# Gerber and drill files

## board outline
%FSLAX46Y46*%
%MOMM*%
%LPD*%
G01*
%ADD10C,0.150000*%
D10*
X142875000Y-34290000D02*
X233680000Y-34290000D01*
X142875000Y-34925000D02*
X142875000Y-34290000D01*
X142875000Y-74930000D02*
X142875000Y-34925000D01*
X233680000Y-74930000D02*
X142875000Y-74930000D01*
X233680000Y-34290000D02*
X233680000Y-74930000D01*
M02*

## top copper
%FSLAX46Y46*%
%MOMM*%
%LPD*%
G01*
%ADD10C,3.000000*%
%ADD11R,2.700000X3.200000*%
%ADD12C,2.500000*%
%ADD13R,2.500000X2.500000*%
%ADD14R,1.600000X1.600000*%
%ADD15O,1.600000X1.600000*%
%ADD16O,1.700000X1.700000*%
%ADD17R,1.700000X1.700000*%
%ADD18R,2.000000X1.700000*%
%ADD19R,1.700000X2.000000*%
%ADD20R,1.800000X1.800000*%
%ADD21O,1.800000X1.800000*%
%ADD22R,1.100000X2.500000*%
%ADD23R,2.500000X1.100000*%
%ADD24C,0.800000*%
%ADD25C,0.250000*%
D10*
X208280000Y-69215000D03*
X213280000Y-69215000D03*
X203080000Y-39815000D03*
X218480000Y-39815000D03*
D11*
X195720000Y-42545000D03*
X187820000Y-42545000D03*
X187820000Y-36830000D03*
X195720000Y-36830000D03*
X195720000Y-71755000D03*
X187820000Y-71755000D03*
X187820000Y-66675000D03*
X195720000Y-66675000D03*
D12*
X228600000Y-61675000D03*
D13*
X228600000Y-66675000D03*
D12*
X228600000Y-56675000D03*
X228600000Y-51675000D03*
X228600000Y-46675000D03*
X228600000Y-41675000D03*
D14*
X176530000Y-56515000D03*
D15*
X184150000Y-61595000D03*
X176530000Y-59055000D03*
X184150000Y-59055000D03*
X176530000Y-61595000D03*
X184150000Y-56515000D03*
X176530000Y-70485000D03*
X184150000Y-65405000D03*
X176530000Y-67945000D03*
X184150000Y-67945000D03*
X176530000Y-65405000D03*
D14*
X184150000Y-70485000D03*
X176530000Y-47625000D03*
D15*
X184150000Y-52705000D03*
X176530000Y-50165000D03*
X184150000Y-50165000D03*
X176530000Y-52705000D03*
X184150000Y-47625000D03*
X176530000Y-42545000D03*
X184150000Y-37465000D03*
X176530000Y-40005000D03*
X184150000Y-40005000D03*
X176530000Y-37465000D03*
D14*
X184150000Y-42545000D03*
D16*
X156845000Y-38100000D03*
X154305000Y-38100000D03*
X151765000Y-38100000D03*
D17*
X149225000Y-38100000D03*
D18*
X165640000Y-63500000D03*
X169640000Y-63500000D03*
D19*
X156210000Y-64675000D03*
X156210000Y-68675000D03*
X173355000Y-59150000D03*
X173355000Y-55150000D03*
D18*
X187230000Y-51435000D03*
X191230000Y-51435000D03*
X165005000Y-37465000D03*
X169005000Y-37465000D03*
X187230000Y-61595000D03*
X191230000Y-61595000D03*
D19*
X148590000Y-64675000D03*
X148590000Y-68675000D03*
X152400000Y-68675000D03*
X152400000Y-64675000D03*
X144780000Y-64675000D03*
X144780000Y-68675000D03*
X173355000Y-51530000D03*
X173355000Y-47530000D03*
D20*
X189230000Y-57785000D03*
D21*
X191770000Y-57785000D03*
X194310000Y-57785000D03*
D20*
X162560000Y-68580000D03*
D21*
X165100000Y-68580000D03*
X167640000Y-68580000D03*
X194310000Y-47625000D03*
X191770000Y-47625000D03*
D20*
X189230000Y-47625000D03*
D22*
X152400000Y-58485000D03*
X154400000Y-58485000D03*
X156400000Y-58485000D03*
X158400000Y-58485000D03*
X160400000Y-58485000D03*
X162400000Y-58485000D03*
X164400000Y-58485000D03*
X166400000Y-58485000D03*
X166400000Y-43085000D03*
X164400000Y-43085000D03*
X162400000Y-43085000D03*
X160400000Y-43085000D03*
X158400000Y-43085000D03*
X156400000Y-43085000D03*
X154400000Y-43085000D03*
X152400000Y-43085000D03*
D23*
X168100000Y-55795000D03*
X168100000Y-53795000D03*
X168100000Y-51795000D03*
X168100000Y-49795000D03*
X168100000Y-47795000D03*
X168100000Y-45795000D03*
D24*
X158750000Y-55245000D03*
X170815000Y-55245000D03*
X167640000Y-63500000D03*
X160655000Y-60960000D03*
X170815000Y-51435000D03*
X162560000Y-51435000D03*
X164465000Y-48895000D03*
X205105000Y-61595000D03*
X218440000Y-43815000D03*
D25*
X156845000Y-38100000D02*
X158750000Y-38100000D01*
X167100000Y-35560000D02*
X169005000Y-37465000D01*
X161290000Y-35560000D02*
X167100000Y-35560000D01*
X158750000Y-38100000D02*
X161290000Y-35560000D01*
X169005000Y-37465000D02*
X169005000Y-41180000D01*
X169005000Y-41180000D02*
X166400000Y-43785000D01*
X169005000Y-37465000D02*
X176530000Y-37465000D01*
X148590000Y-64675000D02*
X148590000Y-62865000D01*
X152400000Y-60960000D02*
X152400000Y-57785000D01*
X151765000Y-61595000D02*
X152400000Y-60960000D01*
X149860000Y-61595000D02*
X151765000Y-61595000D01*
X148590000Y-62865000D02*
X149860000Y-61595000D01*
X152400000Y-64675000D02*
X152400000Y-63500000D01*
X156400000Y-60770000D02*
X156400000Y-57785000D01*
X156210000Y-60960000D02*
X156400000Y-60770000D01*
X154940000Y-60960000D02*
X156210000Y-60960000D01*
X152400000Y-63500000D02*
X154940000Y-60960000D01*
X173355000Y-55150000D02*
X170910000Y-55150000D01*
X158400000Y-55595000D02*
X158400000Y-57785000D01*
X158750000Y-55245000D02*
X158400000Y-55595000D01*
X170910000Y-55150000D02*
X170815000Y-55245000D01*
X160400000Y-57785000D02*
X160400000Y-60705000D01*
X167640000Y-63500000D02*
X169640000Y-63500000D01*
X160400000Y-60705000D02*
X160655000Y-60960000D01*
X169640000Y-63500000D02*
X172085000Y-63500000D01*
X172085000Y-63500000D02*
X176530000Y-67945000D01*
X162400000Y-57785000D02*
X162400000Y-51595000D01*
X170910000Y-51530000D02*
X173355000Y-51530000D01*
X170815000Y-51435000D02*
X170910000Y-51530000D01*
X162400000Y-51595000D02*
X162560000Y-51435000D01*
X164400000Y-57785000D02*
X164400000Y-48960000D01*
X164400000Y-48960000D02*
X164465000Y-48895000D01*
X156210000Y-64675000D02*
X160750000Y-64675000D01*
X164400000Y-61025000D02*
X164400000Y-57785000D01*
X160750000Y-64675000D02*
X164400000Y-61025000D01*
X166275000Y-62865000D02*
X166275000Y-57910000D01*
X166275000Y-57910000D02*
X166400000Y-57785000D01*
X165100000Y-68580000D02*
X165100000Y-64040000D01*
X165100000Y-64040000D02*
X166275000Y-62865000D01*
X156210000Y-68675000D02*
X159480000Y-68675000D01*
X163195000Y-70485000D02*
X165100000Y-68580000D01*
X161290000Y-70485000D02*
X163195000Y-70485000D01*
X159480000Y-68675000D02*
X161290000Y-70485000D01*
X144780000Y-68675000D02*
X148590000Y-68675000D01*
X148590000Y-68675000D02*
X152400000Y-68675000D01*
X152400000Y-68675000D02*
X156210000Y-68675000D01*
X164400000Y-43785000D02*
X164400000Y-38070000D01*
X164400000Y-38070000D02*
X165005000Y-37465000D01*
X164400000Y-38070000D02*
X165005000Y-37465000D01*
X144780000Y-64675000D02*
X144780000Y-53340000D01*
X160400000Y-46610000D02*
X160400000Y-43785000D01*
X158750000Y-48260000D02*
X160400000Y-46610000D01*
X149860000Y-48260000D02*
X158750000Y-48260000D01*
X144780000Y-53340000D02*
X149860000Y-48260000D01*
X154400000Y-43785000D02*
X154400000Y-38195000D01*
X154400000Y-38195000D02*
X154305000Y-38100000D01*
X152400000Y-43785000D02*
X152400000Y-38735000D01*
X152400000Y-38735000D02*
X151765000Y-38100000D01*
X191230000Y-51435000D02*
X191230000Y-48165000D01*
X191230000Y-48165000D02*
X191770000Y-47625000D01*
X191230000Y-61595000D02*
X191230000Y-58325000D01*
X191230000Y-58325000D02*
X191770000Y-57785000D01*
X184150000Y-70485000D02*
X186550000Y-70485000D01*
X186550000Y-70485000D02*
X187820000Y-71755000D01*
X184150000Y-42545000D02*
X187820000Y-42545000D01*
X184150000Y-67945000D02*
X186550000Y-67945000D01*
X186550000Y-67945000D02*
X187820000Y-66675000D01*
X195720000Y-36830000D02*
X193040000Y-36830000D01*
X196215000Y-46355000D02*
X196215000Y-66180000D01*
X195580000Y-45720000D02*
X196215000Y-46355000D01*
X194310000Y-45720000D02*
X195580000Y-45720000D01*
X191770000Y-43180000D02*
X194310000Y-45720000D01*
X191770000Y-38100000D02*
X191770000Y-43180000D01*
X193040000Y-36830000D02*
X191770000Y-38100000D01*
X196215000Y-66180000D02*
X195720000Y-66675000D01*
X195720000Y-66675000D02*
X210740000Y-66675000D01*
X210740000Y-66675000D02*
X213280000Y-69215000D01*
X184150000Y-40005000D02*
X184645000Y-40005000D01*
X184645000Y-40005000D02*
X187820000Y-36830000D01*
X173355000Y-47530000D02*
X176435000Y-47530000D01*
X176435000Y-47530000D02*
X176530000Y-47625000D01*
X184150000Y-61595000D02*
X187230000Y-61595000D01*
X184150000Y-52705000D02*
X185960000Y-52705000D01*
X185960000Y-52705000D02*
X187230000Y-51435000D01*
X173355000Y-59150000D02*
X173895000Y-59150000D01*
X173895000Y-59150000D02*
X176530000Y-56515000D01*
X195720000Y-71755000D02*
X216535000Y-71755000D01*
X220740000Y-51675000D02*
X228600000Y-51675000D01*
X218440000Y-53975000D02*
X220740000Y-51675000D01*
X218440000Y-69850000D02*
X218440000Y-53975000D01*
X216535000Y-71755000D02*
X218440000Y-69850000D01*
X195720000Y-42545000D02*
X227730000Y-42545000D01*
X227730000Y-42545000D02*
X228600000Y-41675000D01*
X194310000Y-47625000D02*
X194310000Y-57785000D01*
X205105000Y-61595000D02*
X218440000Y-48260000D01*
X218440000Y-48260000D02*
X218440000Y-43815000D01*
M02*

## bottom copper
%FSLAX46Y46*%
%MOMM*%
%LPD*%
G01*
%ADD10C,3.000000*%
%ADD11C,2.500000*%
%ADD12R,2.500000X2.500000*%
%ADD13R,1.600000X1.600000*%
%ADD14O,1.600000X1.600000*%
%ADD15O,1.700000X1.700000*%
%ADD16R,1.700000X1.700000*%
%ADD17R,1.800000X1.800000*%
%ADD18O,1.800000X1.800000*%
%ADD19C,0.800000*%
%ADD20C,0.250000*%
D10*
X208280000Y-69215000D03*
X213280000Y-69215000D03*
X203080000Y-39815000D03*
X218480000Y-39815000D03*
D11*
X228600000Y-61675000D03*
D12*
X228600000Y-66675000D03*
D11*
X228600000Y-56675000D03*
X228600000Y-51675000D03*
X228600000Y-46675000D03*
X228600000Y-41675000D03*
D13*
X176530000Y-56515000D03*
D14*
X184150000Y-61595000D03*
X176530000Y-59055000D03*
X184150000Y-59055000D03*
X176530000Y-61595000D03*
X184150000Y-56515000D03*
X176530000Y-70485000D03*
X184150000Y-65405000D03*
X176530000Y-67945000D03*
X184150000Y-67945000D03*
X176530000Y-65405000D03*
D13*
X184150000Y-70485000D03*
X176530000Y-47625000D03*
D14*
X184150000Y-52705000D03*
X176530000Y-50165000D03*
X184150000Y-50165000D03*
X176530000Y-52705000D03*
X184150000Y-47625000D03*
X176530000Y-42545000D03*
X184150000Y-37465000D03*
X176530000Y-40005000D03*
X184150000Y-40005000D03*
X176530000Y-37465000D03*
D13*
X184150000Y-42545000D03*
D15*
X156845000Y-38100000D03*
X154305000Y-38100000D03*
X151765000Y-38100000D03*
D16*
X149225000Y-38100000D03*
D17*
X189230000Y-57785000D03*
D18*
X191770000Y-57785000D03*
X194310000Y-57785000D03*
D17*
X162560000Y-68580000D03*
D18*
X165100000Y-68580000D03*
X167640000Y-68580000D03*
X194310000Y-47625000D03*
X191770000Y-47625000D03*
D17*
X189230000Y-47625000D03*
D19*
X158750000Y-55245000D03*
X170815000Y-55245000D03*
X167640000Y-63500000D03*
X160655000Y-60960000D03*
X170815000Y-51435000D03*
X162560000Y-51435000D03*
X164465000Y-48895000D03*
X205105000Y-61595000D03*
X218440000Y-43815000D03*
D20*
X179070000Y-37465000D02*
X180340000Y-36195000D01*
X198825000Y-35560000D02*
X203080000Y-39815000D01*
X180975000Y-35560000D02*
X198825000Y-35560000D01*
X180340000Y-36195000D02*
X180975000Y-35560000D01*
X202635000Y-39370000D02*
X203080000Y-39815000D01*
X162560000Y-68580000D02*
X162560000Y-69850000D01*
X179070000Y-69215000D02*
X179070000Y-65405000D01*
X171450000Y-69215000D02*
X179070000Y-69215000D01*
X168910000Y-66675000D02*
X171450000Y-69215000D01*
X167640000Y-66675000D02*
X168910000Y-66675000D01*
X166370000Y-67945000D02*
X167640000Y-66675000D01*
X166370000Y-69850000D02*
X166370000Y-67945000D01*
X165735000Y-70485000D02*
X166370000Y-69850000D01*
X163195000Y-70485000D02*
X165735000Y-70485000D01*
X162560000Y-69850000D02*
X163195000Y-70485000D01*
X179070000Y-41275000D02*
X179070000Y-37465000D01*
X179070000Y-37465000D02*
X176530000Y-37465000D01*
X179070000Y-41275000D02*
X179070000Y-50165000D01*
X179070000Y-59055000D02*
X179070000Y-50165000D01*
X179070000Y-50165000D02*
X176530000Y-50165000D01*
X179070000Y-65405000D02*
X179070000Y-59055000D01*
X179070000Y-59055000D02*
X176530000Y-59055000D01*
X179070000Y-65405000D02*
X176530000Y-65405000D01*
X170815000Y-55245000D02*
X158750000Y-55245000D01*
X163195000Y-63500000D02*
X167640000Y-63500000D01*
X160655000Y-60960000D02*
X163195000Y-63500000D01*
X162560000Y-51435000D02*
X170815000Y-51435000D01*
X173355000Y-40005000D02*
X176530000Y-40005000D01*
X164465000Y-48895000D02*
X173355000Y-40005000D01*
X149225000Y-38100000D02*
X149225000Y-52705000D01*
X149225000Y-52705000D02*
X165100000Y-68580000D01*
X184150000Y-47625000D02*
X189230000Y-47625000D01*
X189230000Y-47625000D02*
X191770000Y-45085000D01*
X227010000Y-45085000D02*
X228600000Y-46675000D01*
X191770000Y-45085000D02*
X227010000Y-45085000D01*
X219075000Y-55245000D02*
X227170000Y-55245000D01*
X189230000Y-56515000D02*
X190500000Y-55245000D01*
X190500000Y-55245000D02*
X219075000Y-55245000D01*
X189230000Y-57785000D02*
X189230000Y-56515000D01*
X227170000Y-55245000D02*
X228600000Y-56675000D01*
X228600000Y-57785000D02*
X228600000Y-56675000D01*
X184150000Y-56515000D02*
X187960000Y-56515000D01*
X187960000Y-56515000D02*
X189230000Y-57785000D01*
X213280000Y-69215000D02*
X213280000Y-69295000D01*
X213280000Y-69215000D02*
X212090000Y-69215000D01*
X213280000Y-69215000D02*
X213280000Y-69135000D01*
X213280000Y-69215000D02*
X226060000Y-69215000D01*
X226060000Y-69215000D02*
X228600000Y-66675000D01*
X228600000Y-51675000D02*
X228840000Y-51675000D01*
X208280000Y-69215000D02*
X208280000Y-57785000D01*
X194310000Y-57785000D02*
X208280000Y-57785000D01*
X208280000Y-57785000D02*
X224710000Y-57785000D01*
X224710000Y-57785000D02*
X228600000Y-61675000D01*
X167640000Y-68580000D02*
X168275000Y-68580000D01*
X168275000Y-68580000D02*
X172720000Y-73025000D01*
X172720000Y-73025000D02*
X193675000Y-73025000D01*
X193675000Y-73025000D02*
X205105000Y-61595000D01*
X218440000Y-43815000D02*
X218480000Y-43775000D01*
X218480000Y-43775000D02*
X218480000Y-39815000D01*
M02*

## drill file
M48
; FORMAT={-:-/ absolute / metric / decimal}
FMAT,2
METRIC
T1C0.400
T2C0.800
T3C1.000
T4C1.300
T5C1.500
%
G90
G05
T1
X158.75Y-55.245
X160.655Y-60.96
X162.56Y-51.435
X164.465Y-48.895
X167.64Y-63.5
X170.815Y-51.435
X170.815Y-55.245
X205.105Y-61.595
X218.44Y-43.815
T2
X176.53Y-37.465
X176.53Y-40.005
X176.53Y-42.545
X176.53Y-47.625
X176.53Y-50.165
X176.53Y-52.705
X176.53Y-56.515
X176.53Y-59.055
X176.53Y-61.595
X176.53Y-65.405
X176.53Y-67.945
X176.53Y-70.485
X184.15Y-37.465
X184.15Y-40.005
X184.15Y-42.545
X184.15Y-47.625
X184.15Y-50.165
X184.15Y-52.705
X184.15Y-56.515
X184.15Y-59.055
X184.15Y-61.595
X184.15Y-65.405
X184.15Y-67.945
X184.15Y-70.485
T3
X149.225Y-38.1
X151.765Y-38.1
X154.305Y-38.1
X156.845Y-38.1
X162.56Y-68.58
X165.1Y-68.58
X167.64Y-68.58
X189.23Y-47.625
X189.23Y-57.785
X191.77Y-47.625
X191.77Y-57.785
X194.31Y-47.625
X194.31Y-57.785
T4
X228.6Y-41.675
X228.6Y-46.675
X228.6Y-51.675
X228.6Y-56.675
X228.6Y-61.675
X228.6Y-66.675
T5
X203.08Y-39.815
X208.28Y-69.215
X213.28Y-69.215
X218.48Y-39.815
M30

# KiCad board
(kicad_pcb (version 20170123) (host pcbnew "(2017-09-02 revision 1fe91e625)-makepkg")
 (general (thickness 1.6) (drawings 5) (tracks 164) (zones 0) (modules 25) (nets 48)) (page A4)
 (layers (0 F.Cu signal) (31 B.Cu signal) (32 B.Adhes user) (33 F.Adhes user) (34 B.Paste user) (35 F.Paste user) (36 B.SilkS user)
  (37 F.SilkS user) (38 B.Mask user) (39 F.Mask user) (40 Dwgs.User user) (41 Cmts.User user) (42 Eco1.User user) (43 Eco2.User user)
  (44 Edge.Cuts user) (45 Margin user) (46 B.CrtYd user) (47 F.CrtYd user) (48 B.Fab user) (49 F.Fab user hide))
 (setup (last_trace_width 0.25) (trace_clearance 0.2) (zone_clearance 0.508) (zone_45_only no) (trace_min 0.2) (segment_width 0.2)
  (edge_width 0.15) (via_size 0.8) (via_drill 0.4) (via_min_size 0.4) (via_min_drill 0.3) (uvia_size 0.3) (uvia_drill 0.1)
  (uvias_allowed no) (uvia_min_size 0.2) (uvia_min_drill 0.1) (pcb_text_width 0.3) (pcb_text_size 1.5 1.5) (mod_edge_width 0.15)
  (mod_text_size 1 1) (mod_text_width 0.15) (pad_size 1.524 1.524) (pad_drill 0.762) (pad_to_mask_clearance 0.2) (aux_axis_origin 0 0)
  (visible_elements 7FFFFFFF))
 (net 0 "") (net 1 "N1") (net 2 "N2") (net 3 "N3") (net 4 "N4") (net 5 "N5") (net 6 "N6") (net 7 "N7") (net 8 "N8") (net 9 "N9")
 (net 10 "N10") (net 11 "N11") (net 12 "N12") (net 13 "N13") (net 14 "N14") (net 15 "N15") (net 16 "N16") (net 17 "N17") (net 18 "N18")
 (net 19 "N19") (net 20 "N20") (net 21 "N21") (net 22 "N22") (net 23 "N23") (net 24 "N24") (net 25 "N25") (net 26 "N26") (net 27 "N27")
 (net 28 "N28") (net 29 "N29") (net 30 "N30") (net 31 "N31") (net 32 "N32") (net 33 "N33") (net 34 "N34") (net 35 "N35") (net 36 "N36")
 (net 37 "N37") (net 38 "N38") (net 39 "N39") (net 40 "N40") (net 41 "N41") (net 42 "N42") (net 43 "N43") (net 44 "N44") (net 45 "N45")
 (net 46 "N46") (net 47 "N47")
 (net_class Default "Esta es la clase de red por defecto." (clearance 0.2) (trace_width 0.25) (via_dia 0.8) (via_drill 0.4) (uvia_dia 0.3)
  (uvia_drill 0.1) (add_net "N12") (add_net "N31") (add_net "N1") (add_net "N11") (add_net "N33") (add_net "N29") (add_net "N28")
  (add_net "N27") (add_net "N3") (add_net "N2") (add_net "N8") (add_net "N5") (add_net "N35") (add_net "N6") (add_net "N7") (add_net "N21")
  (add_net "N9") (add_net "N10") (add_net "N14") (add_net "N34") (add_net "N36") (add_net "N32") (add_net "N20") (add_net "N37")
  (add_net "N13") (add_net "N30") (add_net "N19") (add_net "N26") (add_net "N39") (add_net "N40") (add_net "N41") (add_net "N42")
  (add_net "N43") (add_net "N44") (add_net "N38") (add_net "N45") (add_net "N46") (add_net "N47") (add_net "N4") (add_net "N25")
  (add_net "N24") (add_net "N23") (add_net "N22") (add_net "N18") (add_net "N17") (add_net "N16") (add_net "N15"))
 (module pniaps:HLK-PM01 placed (layer F.Cu) (at 208.28 69.215 90)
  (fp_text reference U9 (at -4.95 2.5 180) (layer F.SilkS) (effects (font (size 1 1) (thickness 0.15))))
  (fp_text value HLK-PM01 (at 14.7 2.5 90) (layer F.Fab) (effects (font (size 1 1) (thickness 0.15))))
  (pad 1 thru_hole circle (at 0 0 90) (size 3 3) (drill 1.5) (layers *.Cu *.Mask F.SilkS) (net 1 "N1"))
  (pad 2 thru_hole circle (at 0 5 90) (size 3 3) (drill 1.5) (layers *.Cu *.Mask F.SilkS) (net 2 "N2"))
  (pad 4 thru_hole circle (at 29.4 -5.2 90) (size 3 3) (drill 1.5) (layers *.Cu *.Mask F.SilkS) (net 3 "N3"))
  (pad 3 thru_hole circle (at 29.4 10.2 90) (size 3 3) (drill 1.5) (layers *.Cu *.Mask F.SilkS) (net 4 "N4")))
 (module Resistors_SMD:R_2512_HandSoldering (layer F.Cu) (at 191.77 42.545 180)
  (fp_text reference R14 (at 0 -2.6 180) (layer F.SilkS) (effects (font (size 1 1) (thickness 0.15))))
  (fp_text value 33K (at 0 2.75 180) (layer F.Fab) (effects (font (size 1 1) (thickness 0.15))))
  (pad 1 smd rect (at -3.95 0 180) (size 2.7 3.2) (layers F.Cu F.Paste F.Mask) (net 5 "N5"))
  (pad 2 smd rect (at 3.95 0 180) (size 2.7 3.2) (layers F.Cu F.Paste F.Mask) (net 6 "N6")))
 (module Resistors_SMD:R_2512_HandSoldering (layer F.Cu) (at 191.77 36.83 180)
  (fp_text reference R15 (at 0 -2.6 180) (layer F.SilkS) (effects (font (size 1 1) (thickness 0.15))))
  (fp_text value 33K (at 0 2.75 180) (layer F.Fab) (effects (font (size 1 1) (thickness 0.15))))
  (pad 2 smd rect (at 3.95 0 180) (size 2.7 3.2) (layers F.Cu F.Paste F.Mask) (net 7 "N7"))
  (pad 1 smd rect (at -3.95 0 180) (size 2.7 3.2) (layers F.Cu F.Paste F.Mask) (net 2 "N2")))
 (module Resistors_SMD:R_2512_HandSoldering (layer F.Cu) (at 191.77 71.755 180)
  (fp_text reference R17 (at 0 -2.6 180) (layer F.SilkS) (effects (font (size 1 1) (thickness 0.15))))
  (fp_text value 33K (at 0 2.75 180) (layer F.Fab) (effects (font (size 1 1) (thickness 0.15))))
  (pad 1 smd rect (at -3.95 0 180) (size 2.7 3.2) (layers F.Cu F.Paste F.Mask) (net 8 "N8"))
  (pad 2 smd rect (at 3.95 0 180) (size 2.7 3.2) (layers F.Cu F.Paste F.Mask) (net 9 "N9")))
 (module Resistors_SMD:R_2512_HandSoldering (layer F.Cu) (at 191.77 66.675 180)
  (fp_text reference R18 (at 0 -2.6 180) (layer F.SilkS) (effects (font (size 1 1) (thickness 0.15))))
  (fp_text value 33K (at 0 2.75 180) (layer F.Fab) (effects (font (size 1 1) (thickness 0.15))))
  (pad 2 smd rect (at 3.95 0 180) (size 2.7 3.2) (layers F.Cu F.Paste F.Mask) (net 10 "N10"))
  (pad 1 smd rect (at -3.95 0 180) (size 2.7 3.2) (layers F.Cu F.Paste F.Mask) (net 2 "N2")))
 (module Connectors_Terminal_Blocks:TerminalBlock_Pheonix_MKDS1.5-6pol (layer F.Cu) (at 228.6 66.675 90)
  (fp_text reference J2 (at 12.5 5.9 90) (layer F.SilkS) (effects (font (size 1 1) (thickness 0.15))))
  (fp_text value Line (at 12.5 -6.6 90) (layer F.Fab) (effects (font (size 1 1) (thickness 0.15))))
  (pad 2 thru_hole circle (at 5 0 90) (size 2.5 2.5) (drill 1.3) (layers *.Cu *.Mask) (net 1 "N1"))
  (pad 1 thru_hole rect (at 0 0 90) (size 2.5 2.5) (drill 1.3) (layers *.Cu *.Mask) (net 2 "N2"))
  (pad 3 thru_hole circle (at 10 0 90) (size 2.5 2.5) (drill 1.3) (layers *.Cu *.Mask) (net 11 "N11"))
  (pad 4 thru_hole circle (at 15 0 90) (size 2.5 2.5) (drill 1.3) (layers *.Cu *.Mask) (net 8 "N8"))
  (pad 5 thru_hole circle (at 20 0 90) (size 2.5 2.5) (drill 1.3) (layers *.Cu *.Mask) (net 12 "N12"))
  (pad 6 thru_hole circle (at 25 0 90) (size 2.5 2.5) (drill 1.3) (layers *.Cu *.Mask) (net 5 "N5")))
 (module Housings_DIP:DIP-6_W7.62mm (layer F.Cu) (at 176.53 56.515)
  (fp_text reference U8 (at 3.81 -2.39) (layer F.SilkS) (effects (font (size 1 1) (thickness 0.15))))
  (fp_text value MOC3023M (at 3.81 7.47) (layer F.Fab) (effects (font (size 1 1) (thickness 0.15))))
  (pad 1 thru_hole rect (at 0 0) (size 1.6 1.6) (drill 0.8) (layers *.Cu *.Mask) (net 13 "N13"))
  (pad 4 thru_hole oval (at 7.62 5.08) (size 1.6 1.6) (drill 0.8) (layers *.Cu *.Mask) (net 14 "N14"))
  (pad 2 thru_hole oval (at 0 2.54) (size 1.6 1.6) (drill 0.8) (layers *.Cu *.Mask) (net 3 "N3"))
  (pad 5 thru_hole oval (at 7.62 2.54) (size 1.6 1.6) (drill 0.8) (layers *.Cu *.Mask) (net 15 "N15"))
  (pad 3 thru_hole oval (at 0 5.08) (size 1.6 1.6) (drill 0.8) (layers *.Cu *.Mask) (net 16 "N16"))
  (pad 6 thru_hole oval (at 7.62 0) (size 1.6 1.6) (drill 0.8) (layers *.Cu *.Mask) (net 11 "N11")))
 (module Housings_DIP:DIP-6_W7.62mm (layer F.Cu) (at 184.15 70.485 180)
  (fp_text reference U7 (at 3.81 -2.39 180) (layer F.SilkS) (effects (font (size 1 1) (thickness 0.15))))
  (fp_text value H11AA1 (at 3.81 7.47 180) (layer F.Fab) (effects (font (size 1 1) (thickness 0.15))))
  (pad 6 thru_hole oval (at 7.62 0 180) (size 1.6 1.6) (drill 0.8) (layers *.Cu *.Mask) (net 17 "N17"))
  (pad 3 thru_hole oval (at 0 5.08 180) (size 1.6 1.6) (drill 0.8) (layers *.Cu *.Mask) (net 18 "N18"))
  (pad 5 thru_hole oval (at 7.62 2.54 180) (size 1.6 1.6) (drill 0.8) (layers *.Cu *.Mask) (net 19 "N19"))
  (pad 2 thru_hole oval (at 0 2.54 180) (size 1.6 1.6) (drill 0.8) (layers *.Cu *.Mask) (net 10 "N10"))
  (pad 4 thru_hole oval (at 7.62 5.08 180) (size 1.6 1.6) (drill 0.8) (layers *.Cu *.Mask) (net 3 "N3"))
  (pad 1 thru_hole rect (at 0 0 180) (size 1.6 1.6) (drill 0.8) (layers *.Cu *.Mask) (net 9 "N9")))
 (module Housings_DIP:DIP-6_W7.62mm (layer F.Cu) (at 176.53 47.625)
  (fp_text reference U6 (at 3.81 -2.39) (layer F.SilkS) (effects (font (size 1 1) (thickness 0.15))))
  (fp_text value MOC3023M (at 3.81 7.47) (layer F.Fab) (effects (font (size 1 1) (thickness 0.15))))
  (pad 1 thru_hole rect (at 0 0) (size 1.6 1.6) (drill 0.8) (layers *.Cu *.Mask) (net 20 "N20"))
  (pad 4 thru_hole oval (at 7.62 5.08) (size 1.6 1.6) (drill 0.8) (layers *.Cu *.Mask) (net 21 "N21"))
  (pad 2 thru_hole oval (at 0 2.54) (size 1.6 1.6) (drill 0.8) (layers *.Cu *.Mask) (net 3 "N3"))
  (pad 5 thru_hole oval (at 7.62 2.54) (size 1.6 1.6) (drill 0.8) (layers *.Cu *.Mask) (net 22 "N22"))
  (pad 3 thru_hole oval (at 0 5.08) (size 1.6 1.6) (drill 0.8) (layers *.Cu *.Mask) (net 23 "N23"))
  (pad 6 thru_hole oval (at 7.62 0) (size 1.6 1.6) (drill 0.8) (layers *.Cu *.Mask) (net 12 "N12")))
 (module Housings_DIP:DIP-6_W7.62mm (layer F.Cu) (at 184.15 42.545 180)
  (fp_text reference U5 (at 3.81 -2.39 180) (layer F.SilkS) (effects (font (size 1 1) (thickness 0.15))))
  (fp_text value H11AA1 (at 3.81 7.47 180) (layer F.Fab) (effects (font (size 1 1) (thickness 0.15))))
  (pad 6 thru_hole oval (at 7.62 0 180) (size 1.6 1.6) (drill 0.8) (layers *.Cu *.Mask) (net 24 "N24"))
  (pad 3 thru_hole oval (at 0 5.08 180) (size 1.6 1.6) (drill 0.8) (layers *.Cu *.Mask) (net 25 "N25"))
  (pad 5 thru_hole oval (at 7.62 2.54 180) (size 1.6 1.6) (drill 0.8) (layers *.Cu *.Mask) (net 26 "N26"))
  (pad 2 thru_hole oval (at 0 2.54 180) (size 1.6 1.6) (drill 0.8) (layers *.Cu *.Mask) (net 7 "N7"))
  (pad 4 thru_hole oval (at 7.62 5.08 180) (size 1.6 1.6) (drill 0.8) (layers *.Cu *.Mask) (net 3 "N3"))
  (pad 1 thru_hole rect (at 0 0 180) (size 1.6 1.6) (drill 0.8) (layers *.Cu *.Mask) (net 6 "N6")))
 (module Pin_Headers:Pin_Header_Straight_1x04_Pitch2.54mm (layer F.Cu) (at 149.225 38.1 90)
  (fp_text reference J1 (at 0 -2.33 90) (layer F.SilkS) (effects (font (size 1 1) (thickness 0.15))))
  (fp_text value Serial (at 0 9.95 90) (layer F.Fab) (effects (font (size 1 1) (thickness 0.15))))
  (pad 4 thru_hole oval (at 0 7.62 90) (size 1.7 1.7) (drill 1) (layers *.Cu *.Mask) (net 3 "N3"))
  (pad 3 thru_hole oval (at 0 5.08 90) (size 1.7 1.7) (drill 1) (layers *.Cu *.Mask) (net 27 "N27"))
  (pad 2 thru_hole oval (at 0 2.54 90) (size 1.7 1.7) (drill 1) (layers *.Cu *.Mask) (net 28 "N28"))
  (pad 1 thru_hole rect (at 0 0 90) (size 1.7 1.7) (drill 1) (layers *.Cu *.Mask) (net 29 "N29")))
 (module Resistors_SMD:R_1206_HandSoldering (layer F.Cu) (at 167.64 63.5 180)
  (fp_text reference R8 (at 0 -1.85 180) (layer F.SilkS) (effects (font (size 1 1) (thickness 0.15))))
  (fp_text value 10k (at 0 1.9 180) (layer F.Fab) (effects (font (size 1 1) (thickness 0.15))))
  (pad 2 smd rect (at 2 0 180) (size 2 1.7) (layers F.Cu F.Paste F.Mask) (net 29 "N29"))
  (pad 1 smd rect (at -2 0 180) (size 2 1.7) (layers F.Cu F.Paste F.Mask) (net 19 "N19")))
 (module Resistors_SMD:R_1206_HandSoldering (layer F.Cu) (at 156.21 66.675 270)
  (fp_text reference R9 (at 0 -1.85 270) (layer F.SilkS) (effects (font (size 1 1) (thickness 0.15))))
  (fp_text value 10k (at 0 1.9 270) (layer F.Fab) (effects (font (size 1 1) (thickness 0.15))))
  (pad 1 smd rect (at -2 0 270) (size 2 1.7) (layers F.Cu F.Paste F.Mask) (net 26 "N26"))
  (pad 2 smd rect (at 2 0 270) (size 2 1.7) (layers F.Cu F.Paste F.Mask) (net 29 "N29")))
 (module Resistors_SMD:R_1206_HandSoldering (layer F.Cu) (at 173.355 57.15 90)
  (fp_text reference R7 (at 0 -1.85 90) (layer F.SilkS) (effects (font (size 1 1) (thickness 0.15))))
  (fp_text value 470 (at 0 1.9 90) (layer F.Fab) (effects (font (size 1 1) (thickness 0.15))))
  (pad 1 smd rect (at -2 0 90) (size 2 1.7) (layers F.Cu F.Paste F.Mask) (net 13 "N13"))
  (pad 2 smd rect (at 2 0 90) (size 2 1.7) (layers F.Cu F.Paste F.Mask) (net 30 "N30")))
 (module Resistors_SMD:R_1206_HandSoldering (layer F.Cu) (at 189.23 51.435 180)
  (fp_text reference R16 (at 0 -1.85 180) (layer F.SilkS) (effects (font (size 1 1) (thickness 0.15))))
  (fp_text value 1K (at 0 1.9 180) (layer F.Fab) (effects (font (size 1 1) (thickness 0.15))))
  (pad 2 smd rect (at 2 0 180) (size 2 1.7) (layers F.Cu F.Paste F.Mask) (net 21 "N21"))
  (pad 1 smd rect (at -2 0 180) (size 2 1.7) (layers F.Cu F.Paste F.Mask) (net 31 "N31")))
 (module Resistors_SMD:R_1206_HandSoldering (layer F.Cu) (at 167.005 37.465)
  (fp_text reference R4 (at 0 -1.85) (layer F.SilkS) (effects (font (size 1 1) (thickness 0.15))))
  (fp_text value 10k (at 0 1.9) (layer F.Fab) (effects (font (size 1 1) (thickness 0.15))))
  (pad 1 smd rect (at -2 0) (size 2 1.7) (layers F.Cu F.Paste F.Mask) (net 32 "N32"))
  (pad 2 smd rect (at 2 0) (size 2 1.7) (layers F.Cu F.Paste F.Mask) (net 3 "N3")))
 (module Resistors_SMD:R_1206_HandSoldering (layer F.Cu) (at 189.23 61.595 180)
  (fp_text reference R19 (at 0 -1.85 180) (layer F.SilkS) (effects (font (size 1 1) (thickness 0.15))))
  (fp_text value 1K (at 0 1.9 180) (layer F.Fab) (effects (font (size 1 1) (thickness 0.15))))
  (pad 2 smd rect (at 2 0 180) (size 2 1.7) (layers F.Cu F.Paste F.Mask) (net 14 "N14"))
  (pad 1 smd rect (at -2 0 180) (size 2 1.7) (layers F.Cu F.Paste F.Mask) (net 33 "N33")))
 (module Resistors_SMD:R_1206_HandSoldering (layer F.Cu) (at 148.59 66.675 270)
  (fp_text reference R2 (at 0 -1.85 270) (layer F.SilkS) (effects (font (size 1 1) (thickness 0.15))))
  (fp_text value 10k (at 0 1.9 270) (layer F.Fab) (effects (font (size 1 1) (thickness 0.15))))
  (pad 1 smd rect (at -2 0 270) (size 2 1.7) (layers F.Cu F.Paste F.Mask) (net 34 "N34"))
  (pad 2 smd rect (at 2 0 270) (size 2 1.7) (layers F.Cu F.Paste F.Mask) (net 29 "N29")))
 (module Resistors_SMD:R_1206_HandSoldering (layer F.Cu) (at 152.4 66.675 270)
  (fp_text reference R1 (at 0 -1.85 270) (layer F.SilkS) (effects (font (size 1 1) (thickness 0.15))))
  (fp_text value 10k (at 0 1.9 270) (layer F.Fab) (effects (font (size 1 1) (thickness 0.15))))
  (pad 2 smd rect (at 2 0 270) (size 2 1.7) (layers F.Cu F.Paste F.Mask) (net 29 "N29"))
  (pad 1 smd rect (at -2 0 270) (size 2 1.7) (layers F.Cu F.Paste F.Mask) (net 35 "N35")))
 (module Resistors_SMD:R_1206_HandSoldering (layer F.Cu) (at 144.78 66.675 270)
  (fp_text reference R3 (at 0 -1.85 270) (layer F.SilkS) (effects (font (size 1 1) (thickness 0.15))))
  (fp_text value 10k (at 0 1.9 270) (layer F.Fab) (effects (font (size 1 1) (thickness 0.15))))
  (pad 1 smd rect (at -2 0 270) (size 2 1.7) (layers F.Cu F.Paste F.Mask) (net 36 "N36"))
  (pad 2 smd rect (at 2 0 270) (size 2 1.7) (layers F.Cu F.Paste F.Mask) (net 29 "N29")))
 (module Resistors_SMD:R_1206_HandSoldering (layer F.Cu) (at 173.355 49.53 270)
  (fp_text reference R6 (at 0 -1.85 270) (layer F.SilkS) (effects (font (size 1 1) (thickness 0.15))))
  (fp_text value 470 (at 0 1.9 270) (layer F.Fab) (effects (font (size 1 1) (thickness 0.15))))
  (pad 2 smd rect (at 2 0 270) (size 2 1.7) (layers F.Cu F.Paste F.Mask) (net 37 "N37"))
  (pad 1 smd rect (at -2 0 270) (size 2 1.7) (layers F.Cu F.Paste F.Mask) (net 20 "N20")))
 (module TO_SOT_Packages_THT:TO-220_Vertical (layer F.Cu) (at 189.23 57.785)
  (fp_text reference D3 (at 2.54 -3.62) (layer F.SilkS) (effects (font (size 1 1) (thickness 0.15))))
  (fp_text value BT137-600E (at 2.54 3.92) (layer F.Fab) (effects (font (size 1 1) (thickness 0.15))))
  (pad 1 thru_hole rect (at 0 0) (size 1.8 1.8) (drill 1) (layers *.Cu *.Mask) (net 11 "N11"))
  (pad 2 thru_hole oval (at 2.54 0) (size 1.8 1.8) (drill 1) (layers *.Cu *.Mask) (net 33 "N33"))
  (pad 3 thru_hole oval (at 5.08 0) (size 1.8 1.8) (drill 1) (layers *.Cu *.Mask) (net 1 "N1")))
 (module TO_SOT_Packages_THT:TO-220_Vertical (layer F.Cu) (at 162.56 68.58)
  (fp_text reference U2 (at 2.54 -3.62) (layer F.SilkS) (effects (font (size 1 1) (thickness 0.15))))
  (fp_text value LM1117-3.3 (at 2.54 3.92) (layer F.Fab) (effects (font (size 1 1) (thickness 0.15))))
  (pad 1 thru_hole rect (at 0 0) (size 1.8 1.8) (drill 1) (layers *.Cu *.Mask) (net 3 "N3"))
  (pad 2 thru_hole oval (at 2.54 0) (size 1.8 1.8) (drill 1) (layers *.Cu *.Mask) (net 29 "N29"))
  (pad 3 thru_hole oval (at 5.08 0) (size 1.8 1.8) (drill 1) (layers *.Cu *.Mask) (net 4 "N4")))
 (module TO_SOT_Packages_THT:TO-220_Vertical (layer F.Cu) (at 189.23 47.625)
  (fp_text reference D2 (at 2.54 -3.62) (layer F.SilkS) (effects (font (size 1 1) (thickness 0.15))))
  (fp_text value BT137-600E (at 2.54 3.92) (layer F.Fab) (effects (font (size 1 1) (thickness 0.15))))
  (pad 3 thru_hole oval (at 5.08 0) (size 1.8 1.8) (drill 1) (layers *.Cu *.Mask) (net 1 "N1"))
  (pad 2 thru_hole oval (at 2.54 0) (size 1.8 1.8) (drill 1) (layers *.Cu *.Mask) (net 31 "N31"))
  (pad 1 thru_hole rect (at 0 0) (size 1.8 1.8) (drill 1) (layers *.Cu *.Mask) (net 12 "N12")))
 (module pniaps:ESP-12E (layer F.Cu) (at 152.4 57.785 90)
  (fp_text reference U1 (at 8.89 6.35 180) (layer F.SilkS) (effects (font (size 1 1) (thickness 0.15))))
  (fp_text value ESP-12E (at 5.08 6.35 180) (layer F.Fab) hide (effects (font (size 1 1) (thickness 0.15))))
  (pad 1 smd rect (at 0 0 90) (size 2.5 1.1) (drill (offset -0.7 0)) (layers F.Cu F.Paste F.Mask) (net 34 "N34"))
  (pad 2 smd rect (at 0 2 90) (size 2.5 1.1) (drill (offset -0.7 0)) (layers F.Cu F.Paste F.Mask) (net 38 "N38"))
  (pad 3 smd rect (at 0 4 90) (size 2.5 1.1) (drill (offset -0.7 0)) (layers F.Cu F.Paste F.Mask) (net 35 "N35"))
  (pad 4 smd rect (at 0 6 90) (size 2.5 1.1) (drill (offset -0.7 0)) (layers F.Cu F.Paste F.Mask) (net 30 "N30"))
  (pad 5 smd rect (at 0 8 90) (size 2.5 1.1) (drill (offset -0.7 0)) (layers F.Cu F.Paste F.Mask) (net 19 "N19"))
  (pad 6 smd rect (at 0 10 90) (size 2.5 1.1) (drill (offset -0.7 0)) (layers F.Cu F.Paste F.Mask) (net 37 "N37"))
  (pad 7 smd rect (at 0 12 90) (size 2.5 1.1) (drill (offset -0.7 0)) (layers F.Cu F.Paste F.Mask) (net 26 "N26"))
  (pad 8 smd rect (at 0 14 90) (size 2.5 1.1) (drill (offset -0.7 0)) (layers F.Cu F.Paste F.Mask) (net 29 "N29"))
  (pad 9 smd rect (at 14 14 90) (size 2.5 1.1) (drill (offset 0.7 0)) (layers F.Cu F.Paste F.Mask) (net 3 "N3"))
  (pad 10 smd rect (at 14 12 90) (size 2.5 1.1) (drill (offset 0.7 0)) (layers F.Cu F.Paste F.Mask) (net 32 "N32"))
  (pad 11 smd rect (at 14 10 90) (size 2.5 1.1) (drill (offset 0.7 0)) (layers F.Cu F.Paste F.Mask) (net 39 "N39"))
  (pad 12 smd rect (at 14 8 90) (size 2.5 1.1) (drill (offset 0.7 0)) (layers F.Cu F.Paste F.Mask) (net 36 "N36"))
  (pad 13 smd rect (at 14 6 90) (size 2.5 1.1) (drill (offset 0.7 0)) (layers F.Cu F.Paste F.Mask) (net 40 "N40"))
  (pad 14 smd rect (at 14 4 90) (size 2.5 1.1) (drill (offset 0.7 0)) (layers F.Cu F.Paste F.Mask) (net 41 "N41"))
  (pad 15 smd rect (at 14 2 90) (size 2.5 1.1) (drill (offset 0.7 0)) (layers F.Cu F.Paste F.Mask) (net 27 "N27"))
  (pad 16 smd rect (at 14 0 90) (size 2.5 1.1) (drill (offset 0.7 0)) (layers F.Cu F.Paste F.Mask) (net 28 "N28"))
  (pad 17 smd rect (at 1.99 15 180) (size 2.5 1.1) (drill (offset -0.7 0)) (layers F.Cu F.Paste F.Mask) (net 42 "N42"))
  (pad 18 smd rect (at 3.99 15 180) (size 2.5 1.1) (drill (offset -0.7 0)) (layers F.Cu F.Paste F.Mask) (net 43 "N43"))
  (pad 19 smd rect (at 5.99 15 180) (size 2.5 1.1) (drill (offset -0.7 0)) (layers F.Cu F.Paste F.Mask) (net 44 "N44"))
  (pad 20 smd rect (at 7.99 15 180) (size 2.5 1.1) (drill (offset -0.7 0)) (layers F.Cu F.Paste F.Mask) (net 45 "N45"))
  (pad 21 smd rect (at 9.99 15 180) (size 2.5 1.1) (drill (offset -0.7 0)) (layers F.Cu F.Paste F.Mask) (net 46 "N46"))
  (pad 22 smd rect (at 11.99 15 180) (size 2.5 1.1) (drill (offset -0.7 0)) (layers F.Cu F.Paste F.Mask) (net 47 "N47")))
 (gr_line (start 142.875 34.29) (end 233.68 34.29) (angle 90) (layer Edge.Cuts) (width 0.15))
 (gr_line (start 142.875 34.925) (end 142.875 34.29) (angle 90) (layer Edge.Cuts) (width 0.15))
 (gr_line (start 142.875 74.93) (end 142.875 34.925) (angle 90) (layer Edge.Cuts) (width 0.15))
 (gr_line (start 233.68 74.93) (end 142.875 74.93) (angle 90) (layer Edge.Cuts) (width 0.15))
 (gr_line (start 233.68 34.29) (end 233.68 74.93) (angle 90) (layer Edge.Cuts) (width 0.15))
 (segment (start 179.07 37.465) (end 180.34 36.195) (width 0.25) (layer B.Cu) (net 3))
 (segment (start 198.825 35.56) (end 203.08 39.815) (width 0.25) (layer B.Cu) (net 3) (status 800000))
 (segment (start 180.975 35.56) (end 198.825 35.56) (width 0.25) (layer B.Cu) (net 3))
 (segment (start 180.34 36.195) (end 180.975 35.56) (width 0.25) (layer B.Cu) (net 3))
 (segment (start 156.845 38.1) (end 158.75 38.1) (width 0.25) (layer F.Cu) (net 3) (status 400000))
 (segment (start 167.1 35.56) (end 169.005 37.465) (width 0.25) (layer F.Cu) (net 3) (status 800000))
 (segment (start 161.29 35.56) (end 167.1 35.56) (width 0.25) (layer F.Cu) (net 3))
 (segment (start 158.75 38.1) (end 161.29 35.56) (width 0.25) (layer F.Cu) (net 3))
 (segment (start 169.005 37.465) (end 169.005 41.18) (width 0.25) (layer F.Cu) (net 3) (status 400000))
 (segment (start 169.005 41.18) (end 166.4 43.785) (width 0.25) (layer F.Cu) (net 3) (status 800000))
 (segment (start 169.005 37.465) (end 176.53 37.465) (width 0.25) (layer F.Cu) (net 3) (status C00000))
 (segment (start 202.635 39.37) (end 203.08 39.815) (width 0.25) (layer B.Cu) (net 3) (status C00000))
 (segment (start 162.56 68.58) (end 162.56 69.85) (width 0.25) (layer B.Cu) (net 3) (status 400000))
 (segment (start 179.07 69.215) (end 179.07 65.405) (width 0.25) (layer B.Cu) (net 3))
 (segment (start 171.45 69.215) (end 179.07 69.215) (width 0.25) (layer B.Cu) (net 3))
 (segment (start 168.91 66.675) (end 171.45 69.215) (width 0.25) (layer B.Cu) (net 3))
 (segment (start 167.64 66.675) (end 168.91 66.675) (width 0.25) (layer B.Cu) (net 3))
 (segment (start 166.37 67.945) (end 167.64 66.675) (width 0.25) (layer B.Cu) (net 3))
 (segment (start 166.37 69.85) (end 166.37 67.945) (width 0.25) (layer B.Cu) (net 3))
 (segment (start 165.735 70.485) (end 166.37 69.85) (width 0.25) (layer B.Cu) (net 3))
 (segment (start 163.195 70.485) (end 165.735 70.485) (width 0.25) (layer B.Cu) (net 3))
 (segment (start 162.56 69.85) (end 163.195 70.485) (width 0.25) (layer B.Cu) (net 3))
 (segment (start 179.07 41.275) (end 179.07 37.465) (width 0.25) (layer B.Cu) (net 3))
 (segment (start 179.07 37.465) (end 176.53 37.465) (width 0.25) (layer B.Cu) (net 3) (status 800000))
 (segment (start 179.07 41.275) (end 179.07 50.165) (width 0.25) (layer B.Cu) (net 3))
 (segment (start 179.07 59.055) (end 179.07 50.165) (width 0.25) (layer B.Cu) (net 3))
 (segment (start 179.07 50.165) (end 176.53 50.165) (width 0.25) (layer B.Cu) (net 3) (status 800000))
 (segment (start 179.07 65.405) (end 179.07 59.055) (width 0.25) (layer B.Cu) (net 3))
 (segment (start 179.07 59.055) (end 176.53 59.055) (width 0.25) (layer B.Cu) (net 3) (status 800000))
 (segment (start 179.07 65.405) (end 176.53 65.405) (width 0.25) (layer B.Cu) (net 3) (status 800000))
 (segment (start 148.59 64.675) (end 148.59 62.865) (width 0.25) (layer F.Cu) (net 34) (status 400000))
 (segment (start 152.4 60.96) (end 152.4 57.785) (width 0.25) (layer F.Cu) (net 34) (status 800000))
 (segment (start 151.765 61.595) (end 152.4 60.96) (width 0.25) (layer F.Cu) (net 34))
 (segment (start 149.86 61.595) (end 151.765 61.595) (width 0.25) (layer F.Cu) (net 34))
 (segment (start 148.59 62.865) (end 149.86 61.595) (width 0.25) (layer F.Cu) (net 34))
 (segment (start 152.4 64.675) (end 152.4 63.5) (width 0.25) (layer F.Cu) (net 35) (status 400000))
 (segment (start 156.4 60.77) (end 156.4 57.785) (width 0.25) (layer F.Cu) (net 35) (status 800000))
 (segment (start 156.21 60.96) (end 156.4 60.77) (width 0.25) (layer F.Cu) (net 35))
 (segment (start 154.94 60.96) (end 156.21 60.96) (width 0.25) (layer F.Cu) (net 35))
 (segment (start 152.4 63.5) (end 154.94 60.96) (width 0.25) (layer F.Cu) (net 35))
 (segment (start 173.355 55.15) (end 170.91 55.15) (width 0.25) (layer F.Cu) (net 30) (status 400000))
 (segment (start 158.4 55.595) (end 158.4 57.785) (width 0.25) (layer F.Cu) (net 30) (status 800000))
 (segment (start 158.75 55.245) (end 158.4 55.595) (width 0.25) (layer F.Cu) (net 30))
 (via (at 158.75 55.245) (size 0.8) (drill 0.4) (layers F.Cu B.Cu) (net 30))
 (segment (start 170.815 55.245) (end 158.75 55.245) (width 0.25) (layer B.Cu) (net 30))
 (via (at 170.815 55.245) (size 0.8) (drill 0.4) (layers F.Cu B.Cu) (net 30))
 (segment (start 170.91 55.15) (end 170.815 55.245) (width 0.25) (layer F.Cu) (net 30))
 (segment (start 160.4 57.785) (end 160.4 60.705) (width 0.25) (layer F.Cu) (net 19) (status 400000))
 (segment (start 167.64 63.5) (end 169.64 63.5) (width 0.25) (layer F.Cu) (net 19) (status 800000))
 (via (at 167.64 63.5) (size 0.8) (drill 0.4) (layers F.Cu B.Cu) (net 19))
 (segment (start 163.195 63.5) (end 167.64 63.5) (width 0.25) (layer B.Cu) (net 19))
 (segment (start 160.655 60.96) (end 163.195 63.5) (width 0.25) (layer B.Cu) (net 19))
 (via (at 160.655 60.96) (size 0.8) (drill 0.4) (layers F.Cu B.Cu) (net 19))
 (segment (start 160.4 60.705) (end 160.655 60.96) (width 0.25) (layer F.Cu) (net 19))
 (segment (start 169.64 63.5) (end 172.085 63.5) (width 0.25) (layer F.Cu) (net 19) (status 400000))
 (segment (start 172.085 63.5) (end 176.53 67.945) (width 0.25) (layer F.Cu) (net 19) (status 800000))
 (segment (start 162.4 57.785) (end 162.4 51.595) (width 0.25) (layer F.Cu) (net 37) (status 400000))
 (segment (start 170.91 51.53) (end 173.355 51.53) (width 0.25) (layer F.Cu) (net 37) (status 800000))
 (segment (start 170.815 51.435) (end 170.91 51.53) (width 0.25) (layer F.Cu) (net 37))
 (via (at 170.815 51.435) (size 0.8) (drill 0.4) (layers F.Cu B.Cu) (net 37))
 (segment (start 162.56 51.435) (end 170.815 51.435) (width 0.25) (layer B.Cu) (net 37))
 (via (at 162.56 51.435) (size 0.8) (drill 0.4) (layers F.Cu B.Cu) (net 37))
 (segment (start 162.4 51.595) (end 162.56 51.435) (width 0.25) (layer F.Cu) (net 37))
 (segment (start 164.4 57.785) (end 164.4 48.96) (width 0.25) (layer F.Cu) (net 26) (status 400000))
 (segment (start 173.355 40.005) (end 176.53 40.005) (width 0.25) (layer B.Cu) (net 26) (status 800000))
 (segment (start 164.465 48.895) (end 173.355 40.005) (width 0.25) (layer B.Cu) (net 26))
 (via (at 164.465 48.895) (size 0.8) (drill 0.4) (layers F.Cu B.Cu) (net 26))
 (segment (start 164.4 48.96) (end 164.465 48.895) (width 0.25) (layer F.Cu) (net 26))
 (segment (start 156.21 64.675) (end 160.75 64.675) (width 0.25) (layer F.Cu) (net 26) (status 400000))
 (segment (start 164.4 61.025) (end 164.4 57.785) (width 0.25) (layer F.Cu) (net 26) (status 800000))
 (segment (start 160.75 64.675) (end 164.4 61.025) (width 0.25) (layer F.Cu) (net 26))
 (segment (start 166.275 62.865) (end 166.275 57.91) (width 0.25) (layer F.Cu) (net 29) (status C00000))
 (segment (start 166.275 57.91) (end 166.4 57.785) (width 0.25) (layer F.Cu) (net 29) (status C00000))
 (segment (start 165.1 68.58) (end 165.1 64.04) (width 0.25) (layer F.Cu) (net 29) (status 400000))
 (segment (start 165.1 64.04) (end 166.275 62.865) (width 0.25) (layer F.Cu) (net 29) (status 800000))
 (segment (start 156.21 68.675) (end 159.48 68.675) (width 0.25) (layer F.Cu) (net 29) (status 400000))
 (segment (start 163.195 70.485) (end 165.1 68.58) (width 0.25) (layer F.Cu) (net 29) (status 800000))
 (segment (start 161.29 70.485) (end 163.195 70.485) (width 0.25) (layer F.Cu) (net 29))
 (segment (start 159.48 68.675) (end 161.29 70.485) (width 0.25) (layer F.Cu) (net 29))
 (segment (start 144.78 68.675) (end 148.59 68.675) (width 0.25) (layer F.Cu) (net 29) (status C00000))
 (segment (start 148.59 68.675) (end 152.4 68.675) (width 0.25) (layer F.Cu) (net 29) (status C00000))
 (segment (start 152.4 68.675) (end 156.21 68.675) (width 0.25) (layer F.Cu) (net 29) (status C00000))
 (segment (start 149.225 38.1) (end 149.225 52.705) (width 0.25) (layer B.Cu) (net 29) (status 400000))
 (segment (start 149.225 52.705) (end 165.1 68.58) (width 0.25) (layer B.Cu) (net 29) (status 800000))
 (segment (start 164.4 43.785) (end 164.4 38.07) (width 0.25) (layer F.Cu) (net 32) (status C00000))
 (segment (start 164.4 38.07) (end 165.005 37.465) (width 0.25) (layer F.Cu) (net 32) (status C00000))
 (segment (start 164.4 38.07) (end 165.005 37.465) (width 0.25) (layer F.Cu) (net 32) (status C00000))
 (segment (start 144.78 64.675) (end 144.78 53.34) (width 0.25) (layer F.Cu) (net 36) (status 400000))
 (segment (start 160.4 46.61) (end 160.4 43.785) (width 0.25) (layer F.Cu) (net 36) (status 800000))
 (segment (start 158.75 48.26) (end 160.4 46.61) (width 0.25) (layer F.Cu) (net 36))
 (segment (start 149.86 48.26) (end 158.75 48.26) (width 0.25) (layer F.Cu) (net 36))
 (segment (start 144.78 53.34) (end 149.86 48.26) (width 0.25) (layer F.Cu) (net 36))
 (segment (start 154.4 43.785) (end 154.4 38.195) (width 0.25) (layer F.Cu) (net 27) (status C00000))
 (segment (start 154.4 38.195) (end 154.305 38.1) (width 0.25) (layer F.Cu) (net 27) (status C00000))
 (segment (start 152.4 43.785) (end 152.4 38.735) (width 0.25) (layer F.Cu) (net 28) (status 400000))
 (segment (start 152.4 38.735) (end 151.765 38.1) (width 0.25) (layer F.Cu) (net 28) (status 800000))
 (segment (start 191.23 51.435) (end 191.23 48.165) (width 0.25) (layer F.Cu) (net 31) (status C00000))
 (segment (start 191.23 48.165) (end 191.77 47.625) (width 0.25) (layer F.Cu) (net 31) (status C00000))
 (segment (start 184.15 47.625) (end 189.23 47.625) (width 0.25) (layer B.Cu) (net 12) (status C00000))
 (segment (start 189.23 47.625) (end 191.77 45.085) (width 0.25) (layer B.Cu) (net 12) (status 400000))
 (segment (start 227.01 45.085) (end 228.6 46.675) (width 0.25) (layer B.Cu) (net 12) (status 800000))
 (segment (start 191.77 45.085) (end 227.01 45.085) (width 0.25) (layer B.Cu) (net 12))
 (segment (start 219.075 55.245) (end 227.17 55.245) (width 0.25) (layer B.Cu) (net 11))
 (segment (start 189.23 56.515) (end 190.5 55.245) (width 0.25) (layer B.Cu) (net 11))
 (segment (start 190.5 55.245) (end 219.075 55.245) (width 0.25) (layer B.Cu) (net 11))
 (segment (start 189.23 57.785) (end 189.23 56.515) (width 0.25) (layer B.Cu) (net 11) (status 400000))
 (segment (start 227.17 55.245) (end 228.6 56.675) (width 0.25) (layer B.Cu) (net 11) (status 800000))
 (segment (start 228.6 57.785) (end 228.6 56.675) (width 0.25) (layer B.Cu) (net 11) (status C00000))
 (segment (start 184.15 56.515) (end 187.96 56.515) (width 0.25) (layer B.Cu) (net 11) (status 400000))
 (segment (start 187.96 56.515) (end 189.23 57.785) (width 0.25) (layer B.Cu) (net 11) (status 800000))
 (segment (start 191.23 61.595) (end 191.23 58.325) (width 0.25) (layer F.Cu) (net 33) (status C00000))
 (segment (start 191.23 58.325) (end 191.77 57.785) (width 0.25) (layer F.Cu) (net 33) (status C00000))
 (segment (start 184.15 70.485) (end 186.55 70.485) (width 0.25) (layer F.Cu) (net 9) (status C00000))
 (segment (start 186.55 70.485) (end 187.82 71.755) (width 0.25) (layer F.Cu) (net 9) (status C00000))
 (segment (start 184.15 42.545) (end 187.82 42.545) (width 0.25) (layer F.Cu) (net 6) (status C00000))
 (segment (start 184.15 67.945) (end 186.55 67.945) (width 0.25) (layer F.Cu) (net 10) (status C00000))
 (segment (start 186.55 67.945) (end 187.82 66.675) (width 0.25) (layer F.Cu) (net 10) (status C00000))
 (segment (start 195.72 36.83) (end 193.04 36.83) (width 0.25) (layer F.Cu) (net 2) (status 400000))
 (segment (start 196.215 46.355) (end 196.215 66.18) (width 0.25) (layer F.Cu) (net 2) (status 800000))
 (segment (start 195.58 45.72) (end 196.215 46.355) (width 0.25) (layer F.Cu) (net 2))
 (segment (start 194.31 45.72) (end 195.58 45.72) (width 0.25) (layer F.Cu) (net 2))
 (segment (start 191.77 43.18) (end 194.31 45.72) (width 0.25) (layer F.Cu) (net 2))
 (segment (start 191.77 38.1) (end 191.77 43.18) (width 0.25) (layer F.Cu) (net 2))
 (segment (start 193.04 36.83) (end 191.77 38.1) (width 0.25) (layer F.Cu) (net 2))
 (segment (start 196.215 66.18) (end 195.72 66.675) (width 0.25) (layer F.Cu) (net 2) (status C00000))
 (segment (start 195.72 66.675) (end 210.74 66.675) (width 0.25) (layer F.Cu) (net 2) (status 400000))
 (segment (start 210.74 66.675) (end 213.28 69.215) (width 0.25) (layer F.Cu) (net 2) (status 800000))
 (segment (start 213.28 69.215) (end 213.28 69.295) (width 0.25) (layer B.Cu) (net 2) (status C00000))
 (segment (start 213.28 69.215) (end 212.09 69.215) (width 0.25) (layer B.Cu) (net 2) (status C00000))
 (segment (start 213.28 69.215) (end 213.28 69.135) (width 0.25) (layer B.Cu) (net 2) (status C00000))
 (segment (start 213.28 69.215) (end 226.06 69.215) (width 0.25) (layer B.Cu) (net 2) (status 400000))
 (segment (start 226.06 69.215) (end 228.6 66.675) (width 0.25) (layer B.Cu) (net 2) (status 800000))
 (segment (start 184.15 40.005) (end 184.645 40.005) (width 0.25) (layer F.Cu) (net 7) (status C00000))
 (segment (start 184.645 40.005) (end 187.82 36.83) (width 0.25) (layer F.Cu) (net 7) (status C00000))
 (segment (start 173.355 47.53) (end 176.435 47.53) (width 0.25) (layer F.Cu) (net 20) (status C00000))
 (segment (start 176.435 47.53) (end 176.53 47.625) (width 0.25) (layer F.Cu) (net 20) (status C00000))
 (segment (start 184.15 61.595) (end 187.23 61.595) (width 0.25) (layer F.Cu) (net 14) (status C00000))
 (segment (start 184.15 52.705) (end 185.96 52.705) (width 0.25) (layer F.Cu) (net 21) (status 400000))
 (segment (start 185.96 52.705) (end 187.23 51.435) (width 0.25) (layer F.Cu) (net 21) (status 800000))
 (segment (start 173.355 59.15) (end 173.895 59.15) (width 0.25) (layer F.Cu) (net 13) (status C00000))
 (segment (start 173.895 59.15) (end 176.53 56.515) (width 0.25) (layer F.Cu) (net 13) (status C00000))
 (segment (start 195.72 71.755) (end 216.535 71.755) (width 0.25) (layer F.Cu) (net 8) (status 400000))
 (segment (start 220.74 51.675) (end 228.6 51.675) (width 0.25) (layer F.Cu) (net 8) (status 800000))
 (segment (start 218.44 53.975) (end 220.74 51.675) (width 0.25) (layer F.Cu) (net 8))
 (segment (start 218.44 69.85) (end 218.44 53.975) (width 0.25) (layer F.Cu) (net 8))
 (segment (start 216.535 71.755) (end 218.44 69.85) (width 0.25) (layer F.Cu) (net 8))
 (segment (start 228.6 51.675) (end 228.84 51.675) (width 0.25) (layer B.Cu) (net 8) (status C00000))
 (segment (start 195.72 42.545) (end 227.73 42.545) (width 0.25) (layer F.Cu) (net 5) (status C00000))
 (segment (start 227.73 42.545) (end 228.6 41.675) (width 0.25) (layer F.Cu) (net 5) (status C00000))
 (segment (start 194.31 47.625) (end 194.31 57.785) (width 0.25) (layer F.Cu) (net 1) (status C00000))
 (segment (start 208.28 69.215) (end 208.28 57.785) (width 0.25) (layer B.Cu) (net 1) (status 400000))
 (segment (start 194.31 57.785) (end 208.28 57.785) (width 0.25) (layer B.Cu) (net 1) (status 400000))
 (segment (start 208.28 57.785) (end 224.71 57.785) (width 0.25) (layer B.Cu) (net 1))
 (segment (start 224.71 57.785) (end 228.6 61.675) (width 0.25) (layer B.Cu) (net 1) (status 800000))
 (segment (start 167.64 68.58) (end 168.275 68.58) (width 0.25) (layer B.Cu) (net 4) (status C00000))
 (segment (start 168.275 68.58) (end 172.72 73.025) (width 0.25) (layer B.Cu) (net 4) (status 400000))
 (segment (start 172.72 73.025) (end 193.675 73.025) (width 0.25) (layer B.Cu) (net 4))
 (segment (start 193.675 73.025) (end 205.105 61.595) (width 0.25) (layer B.Cu) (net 4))
 (via (at 205.105 61.595) (size 0.8) (drill 0.4) (layers F.Cu B.Cu) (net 4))
 (segment (start 205.105 61.595) (end 218.44 48.26) (width 0.25) (layer F.Cu) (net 4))
 (segment (start 218.44 48.26) (end 218.44 43.815) (width 0.25) (layer F.Cu) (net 4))
 (via (at 218.44 43.815) (size 0.8) (drill 0.4) (layers F.Cu B.Cu) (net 4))
 (segment (start 218.44 43.815) (end 218.48 43.775) (width 0.25) (layer B.Cu) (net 4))
 (segment (start 218.48 43.775) (end 218.48 39.815) (width 0.25) (layer B.Cu) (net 4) (status 800000)))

